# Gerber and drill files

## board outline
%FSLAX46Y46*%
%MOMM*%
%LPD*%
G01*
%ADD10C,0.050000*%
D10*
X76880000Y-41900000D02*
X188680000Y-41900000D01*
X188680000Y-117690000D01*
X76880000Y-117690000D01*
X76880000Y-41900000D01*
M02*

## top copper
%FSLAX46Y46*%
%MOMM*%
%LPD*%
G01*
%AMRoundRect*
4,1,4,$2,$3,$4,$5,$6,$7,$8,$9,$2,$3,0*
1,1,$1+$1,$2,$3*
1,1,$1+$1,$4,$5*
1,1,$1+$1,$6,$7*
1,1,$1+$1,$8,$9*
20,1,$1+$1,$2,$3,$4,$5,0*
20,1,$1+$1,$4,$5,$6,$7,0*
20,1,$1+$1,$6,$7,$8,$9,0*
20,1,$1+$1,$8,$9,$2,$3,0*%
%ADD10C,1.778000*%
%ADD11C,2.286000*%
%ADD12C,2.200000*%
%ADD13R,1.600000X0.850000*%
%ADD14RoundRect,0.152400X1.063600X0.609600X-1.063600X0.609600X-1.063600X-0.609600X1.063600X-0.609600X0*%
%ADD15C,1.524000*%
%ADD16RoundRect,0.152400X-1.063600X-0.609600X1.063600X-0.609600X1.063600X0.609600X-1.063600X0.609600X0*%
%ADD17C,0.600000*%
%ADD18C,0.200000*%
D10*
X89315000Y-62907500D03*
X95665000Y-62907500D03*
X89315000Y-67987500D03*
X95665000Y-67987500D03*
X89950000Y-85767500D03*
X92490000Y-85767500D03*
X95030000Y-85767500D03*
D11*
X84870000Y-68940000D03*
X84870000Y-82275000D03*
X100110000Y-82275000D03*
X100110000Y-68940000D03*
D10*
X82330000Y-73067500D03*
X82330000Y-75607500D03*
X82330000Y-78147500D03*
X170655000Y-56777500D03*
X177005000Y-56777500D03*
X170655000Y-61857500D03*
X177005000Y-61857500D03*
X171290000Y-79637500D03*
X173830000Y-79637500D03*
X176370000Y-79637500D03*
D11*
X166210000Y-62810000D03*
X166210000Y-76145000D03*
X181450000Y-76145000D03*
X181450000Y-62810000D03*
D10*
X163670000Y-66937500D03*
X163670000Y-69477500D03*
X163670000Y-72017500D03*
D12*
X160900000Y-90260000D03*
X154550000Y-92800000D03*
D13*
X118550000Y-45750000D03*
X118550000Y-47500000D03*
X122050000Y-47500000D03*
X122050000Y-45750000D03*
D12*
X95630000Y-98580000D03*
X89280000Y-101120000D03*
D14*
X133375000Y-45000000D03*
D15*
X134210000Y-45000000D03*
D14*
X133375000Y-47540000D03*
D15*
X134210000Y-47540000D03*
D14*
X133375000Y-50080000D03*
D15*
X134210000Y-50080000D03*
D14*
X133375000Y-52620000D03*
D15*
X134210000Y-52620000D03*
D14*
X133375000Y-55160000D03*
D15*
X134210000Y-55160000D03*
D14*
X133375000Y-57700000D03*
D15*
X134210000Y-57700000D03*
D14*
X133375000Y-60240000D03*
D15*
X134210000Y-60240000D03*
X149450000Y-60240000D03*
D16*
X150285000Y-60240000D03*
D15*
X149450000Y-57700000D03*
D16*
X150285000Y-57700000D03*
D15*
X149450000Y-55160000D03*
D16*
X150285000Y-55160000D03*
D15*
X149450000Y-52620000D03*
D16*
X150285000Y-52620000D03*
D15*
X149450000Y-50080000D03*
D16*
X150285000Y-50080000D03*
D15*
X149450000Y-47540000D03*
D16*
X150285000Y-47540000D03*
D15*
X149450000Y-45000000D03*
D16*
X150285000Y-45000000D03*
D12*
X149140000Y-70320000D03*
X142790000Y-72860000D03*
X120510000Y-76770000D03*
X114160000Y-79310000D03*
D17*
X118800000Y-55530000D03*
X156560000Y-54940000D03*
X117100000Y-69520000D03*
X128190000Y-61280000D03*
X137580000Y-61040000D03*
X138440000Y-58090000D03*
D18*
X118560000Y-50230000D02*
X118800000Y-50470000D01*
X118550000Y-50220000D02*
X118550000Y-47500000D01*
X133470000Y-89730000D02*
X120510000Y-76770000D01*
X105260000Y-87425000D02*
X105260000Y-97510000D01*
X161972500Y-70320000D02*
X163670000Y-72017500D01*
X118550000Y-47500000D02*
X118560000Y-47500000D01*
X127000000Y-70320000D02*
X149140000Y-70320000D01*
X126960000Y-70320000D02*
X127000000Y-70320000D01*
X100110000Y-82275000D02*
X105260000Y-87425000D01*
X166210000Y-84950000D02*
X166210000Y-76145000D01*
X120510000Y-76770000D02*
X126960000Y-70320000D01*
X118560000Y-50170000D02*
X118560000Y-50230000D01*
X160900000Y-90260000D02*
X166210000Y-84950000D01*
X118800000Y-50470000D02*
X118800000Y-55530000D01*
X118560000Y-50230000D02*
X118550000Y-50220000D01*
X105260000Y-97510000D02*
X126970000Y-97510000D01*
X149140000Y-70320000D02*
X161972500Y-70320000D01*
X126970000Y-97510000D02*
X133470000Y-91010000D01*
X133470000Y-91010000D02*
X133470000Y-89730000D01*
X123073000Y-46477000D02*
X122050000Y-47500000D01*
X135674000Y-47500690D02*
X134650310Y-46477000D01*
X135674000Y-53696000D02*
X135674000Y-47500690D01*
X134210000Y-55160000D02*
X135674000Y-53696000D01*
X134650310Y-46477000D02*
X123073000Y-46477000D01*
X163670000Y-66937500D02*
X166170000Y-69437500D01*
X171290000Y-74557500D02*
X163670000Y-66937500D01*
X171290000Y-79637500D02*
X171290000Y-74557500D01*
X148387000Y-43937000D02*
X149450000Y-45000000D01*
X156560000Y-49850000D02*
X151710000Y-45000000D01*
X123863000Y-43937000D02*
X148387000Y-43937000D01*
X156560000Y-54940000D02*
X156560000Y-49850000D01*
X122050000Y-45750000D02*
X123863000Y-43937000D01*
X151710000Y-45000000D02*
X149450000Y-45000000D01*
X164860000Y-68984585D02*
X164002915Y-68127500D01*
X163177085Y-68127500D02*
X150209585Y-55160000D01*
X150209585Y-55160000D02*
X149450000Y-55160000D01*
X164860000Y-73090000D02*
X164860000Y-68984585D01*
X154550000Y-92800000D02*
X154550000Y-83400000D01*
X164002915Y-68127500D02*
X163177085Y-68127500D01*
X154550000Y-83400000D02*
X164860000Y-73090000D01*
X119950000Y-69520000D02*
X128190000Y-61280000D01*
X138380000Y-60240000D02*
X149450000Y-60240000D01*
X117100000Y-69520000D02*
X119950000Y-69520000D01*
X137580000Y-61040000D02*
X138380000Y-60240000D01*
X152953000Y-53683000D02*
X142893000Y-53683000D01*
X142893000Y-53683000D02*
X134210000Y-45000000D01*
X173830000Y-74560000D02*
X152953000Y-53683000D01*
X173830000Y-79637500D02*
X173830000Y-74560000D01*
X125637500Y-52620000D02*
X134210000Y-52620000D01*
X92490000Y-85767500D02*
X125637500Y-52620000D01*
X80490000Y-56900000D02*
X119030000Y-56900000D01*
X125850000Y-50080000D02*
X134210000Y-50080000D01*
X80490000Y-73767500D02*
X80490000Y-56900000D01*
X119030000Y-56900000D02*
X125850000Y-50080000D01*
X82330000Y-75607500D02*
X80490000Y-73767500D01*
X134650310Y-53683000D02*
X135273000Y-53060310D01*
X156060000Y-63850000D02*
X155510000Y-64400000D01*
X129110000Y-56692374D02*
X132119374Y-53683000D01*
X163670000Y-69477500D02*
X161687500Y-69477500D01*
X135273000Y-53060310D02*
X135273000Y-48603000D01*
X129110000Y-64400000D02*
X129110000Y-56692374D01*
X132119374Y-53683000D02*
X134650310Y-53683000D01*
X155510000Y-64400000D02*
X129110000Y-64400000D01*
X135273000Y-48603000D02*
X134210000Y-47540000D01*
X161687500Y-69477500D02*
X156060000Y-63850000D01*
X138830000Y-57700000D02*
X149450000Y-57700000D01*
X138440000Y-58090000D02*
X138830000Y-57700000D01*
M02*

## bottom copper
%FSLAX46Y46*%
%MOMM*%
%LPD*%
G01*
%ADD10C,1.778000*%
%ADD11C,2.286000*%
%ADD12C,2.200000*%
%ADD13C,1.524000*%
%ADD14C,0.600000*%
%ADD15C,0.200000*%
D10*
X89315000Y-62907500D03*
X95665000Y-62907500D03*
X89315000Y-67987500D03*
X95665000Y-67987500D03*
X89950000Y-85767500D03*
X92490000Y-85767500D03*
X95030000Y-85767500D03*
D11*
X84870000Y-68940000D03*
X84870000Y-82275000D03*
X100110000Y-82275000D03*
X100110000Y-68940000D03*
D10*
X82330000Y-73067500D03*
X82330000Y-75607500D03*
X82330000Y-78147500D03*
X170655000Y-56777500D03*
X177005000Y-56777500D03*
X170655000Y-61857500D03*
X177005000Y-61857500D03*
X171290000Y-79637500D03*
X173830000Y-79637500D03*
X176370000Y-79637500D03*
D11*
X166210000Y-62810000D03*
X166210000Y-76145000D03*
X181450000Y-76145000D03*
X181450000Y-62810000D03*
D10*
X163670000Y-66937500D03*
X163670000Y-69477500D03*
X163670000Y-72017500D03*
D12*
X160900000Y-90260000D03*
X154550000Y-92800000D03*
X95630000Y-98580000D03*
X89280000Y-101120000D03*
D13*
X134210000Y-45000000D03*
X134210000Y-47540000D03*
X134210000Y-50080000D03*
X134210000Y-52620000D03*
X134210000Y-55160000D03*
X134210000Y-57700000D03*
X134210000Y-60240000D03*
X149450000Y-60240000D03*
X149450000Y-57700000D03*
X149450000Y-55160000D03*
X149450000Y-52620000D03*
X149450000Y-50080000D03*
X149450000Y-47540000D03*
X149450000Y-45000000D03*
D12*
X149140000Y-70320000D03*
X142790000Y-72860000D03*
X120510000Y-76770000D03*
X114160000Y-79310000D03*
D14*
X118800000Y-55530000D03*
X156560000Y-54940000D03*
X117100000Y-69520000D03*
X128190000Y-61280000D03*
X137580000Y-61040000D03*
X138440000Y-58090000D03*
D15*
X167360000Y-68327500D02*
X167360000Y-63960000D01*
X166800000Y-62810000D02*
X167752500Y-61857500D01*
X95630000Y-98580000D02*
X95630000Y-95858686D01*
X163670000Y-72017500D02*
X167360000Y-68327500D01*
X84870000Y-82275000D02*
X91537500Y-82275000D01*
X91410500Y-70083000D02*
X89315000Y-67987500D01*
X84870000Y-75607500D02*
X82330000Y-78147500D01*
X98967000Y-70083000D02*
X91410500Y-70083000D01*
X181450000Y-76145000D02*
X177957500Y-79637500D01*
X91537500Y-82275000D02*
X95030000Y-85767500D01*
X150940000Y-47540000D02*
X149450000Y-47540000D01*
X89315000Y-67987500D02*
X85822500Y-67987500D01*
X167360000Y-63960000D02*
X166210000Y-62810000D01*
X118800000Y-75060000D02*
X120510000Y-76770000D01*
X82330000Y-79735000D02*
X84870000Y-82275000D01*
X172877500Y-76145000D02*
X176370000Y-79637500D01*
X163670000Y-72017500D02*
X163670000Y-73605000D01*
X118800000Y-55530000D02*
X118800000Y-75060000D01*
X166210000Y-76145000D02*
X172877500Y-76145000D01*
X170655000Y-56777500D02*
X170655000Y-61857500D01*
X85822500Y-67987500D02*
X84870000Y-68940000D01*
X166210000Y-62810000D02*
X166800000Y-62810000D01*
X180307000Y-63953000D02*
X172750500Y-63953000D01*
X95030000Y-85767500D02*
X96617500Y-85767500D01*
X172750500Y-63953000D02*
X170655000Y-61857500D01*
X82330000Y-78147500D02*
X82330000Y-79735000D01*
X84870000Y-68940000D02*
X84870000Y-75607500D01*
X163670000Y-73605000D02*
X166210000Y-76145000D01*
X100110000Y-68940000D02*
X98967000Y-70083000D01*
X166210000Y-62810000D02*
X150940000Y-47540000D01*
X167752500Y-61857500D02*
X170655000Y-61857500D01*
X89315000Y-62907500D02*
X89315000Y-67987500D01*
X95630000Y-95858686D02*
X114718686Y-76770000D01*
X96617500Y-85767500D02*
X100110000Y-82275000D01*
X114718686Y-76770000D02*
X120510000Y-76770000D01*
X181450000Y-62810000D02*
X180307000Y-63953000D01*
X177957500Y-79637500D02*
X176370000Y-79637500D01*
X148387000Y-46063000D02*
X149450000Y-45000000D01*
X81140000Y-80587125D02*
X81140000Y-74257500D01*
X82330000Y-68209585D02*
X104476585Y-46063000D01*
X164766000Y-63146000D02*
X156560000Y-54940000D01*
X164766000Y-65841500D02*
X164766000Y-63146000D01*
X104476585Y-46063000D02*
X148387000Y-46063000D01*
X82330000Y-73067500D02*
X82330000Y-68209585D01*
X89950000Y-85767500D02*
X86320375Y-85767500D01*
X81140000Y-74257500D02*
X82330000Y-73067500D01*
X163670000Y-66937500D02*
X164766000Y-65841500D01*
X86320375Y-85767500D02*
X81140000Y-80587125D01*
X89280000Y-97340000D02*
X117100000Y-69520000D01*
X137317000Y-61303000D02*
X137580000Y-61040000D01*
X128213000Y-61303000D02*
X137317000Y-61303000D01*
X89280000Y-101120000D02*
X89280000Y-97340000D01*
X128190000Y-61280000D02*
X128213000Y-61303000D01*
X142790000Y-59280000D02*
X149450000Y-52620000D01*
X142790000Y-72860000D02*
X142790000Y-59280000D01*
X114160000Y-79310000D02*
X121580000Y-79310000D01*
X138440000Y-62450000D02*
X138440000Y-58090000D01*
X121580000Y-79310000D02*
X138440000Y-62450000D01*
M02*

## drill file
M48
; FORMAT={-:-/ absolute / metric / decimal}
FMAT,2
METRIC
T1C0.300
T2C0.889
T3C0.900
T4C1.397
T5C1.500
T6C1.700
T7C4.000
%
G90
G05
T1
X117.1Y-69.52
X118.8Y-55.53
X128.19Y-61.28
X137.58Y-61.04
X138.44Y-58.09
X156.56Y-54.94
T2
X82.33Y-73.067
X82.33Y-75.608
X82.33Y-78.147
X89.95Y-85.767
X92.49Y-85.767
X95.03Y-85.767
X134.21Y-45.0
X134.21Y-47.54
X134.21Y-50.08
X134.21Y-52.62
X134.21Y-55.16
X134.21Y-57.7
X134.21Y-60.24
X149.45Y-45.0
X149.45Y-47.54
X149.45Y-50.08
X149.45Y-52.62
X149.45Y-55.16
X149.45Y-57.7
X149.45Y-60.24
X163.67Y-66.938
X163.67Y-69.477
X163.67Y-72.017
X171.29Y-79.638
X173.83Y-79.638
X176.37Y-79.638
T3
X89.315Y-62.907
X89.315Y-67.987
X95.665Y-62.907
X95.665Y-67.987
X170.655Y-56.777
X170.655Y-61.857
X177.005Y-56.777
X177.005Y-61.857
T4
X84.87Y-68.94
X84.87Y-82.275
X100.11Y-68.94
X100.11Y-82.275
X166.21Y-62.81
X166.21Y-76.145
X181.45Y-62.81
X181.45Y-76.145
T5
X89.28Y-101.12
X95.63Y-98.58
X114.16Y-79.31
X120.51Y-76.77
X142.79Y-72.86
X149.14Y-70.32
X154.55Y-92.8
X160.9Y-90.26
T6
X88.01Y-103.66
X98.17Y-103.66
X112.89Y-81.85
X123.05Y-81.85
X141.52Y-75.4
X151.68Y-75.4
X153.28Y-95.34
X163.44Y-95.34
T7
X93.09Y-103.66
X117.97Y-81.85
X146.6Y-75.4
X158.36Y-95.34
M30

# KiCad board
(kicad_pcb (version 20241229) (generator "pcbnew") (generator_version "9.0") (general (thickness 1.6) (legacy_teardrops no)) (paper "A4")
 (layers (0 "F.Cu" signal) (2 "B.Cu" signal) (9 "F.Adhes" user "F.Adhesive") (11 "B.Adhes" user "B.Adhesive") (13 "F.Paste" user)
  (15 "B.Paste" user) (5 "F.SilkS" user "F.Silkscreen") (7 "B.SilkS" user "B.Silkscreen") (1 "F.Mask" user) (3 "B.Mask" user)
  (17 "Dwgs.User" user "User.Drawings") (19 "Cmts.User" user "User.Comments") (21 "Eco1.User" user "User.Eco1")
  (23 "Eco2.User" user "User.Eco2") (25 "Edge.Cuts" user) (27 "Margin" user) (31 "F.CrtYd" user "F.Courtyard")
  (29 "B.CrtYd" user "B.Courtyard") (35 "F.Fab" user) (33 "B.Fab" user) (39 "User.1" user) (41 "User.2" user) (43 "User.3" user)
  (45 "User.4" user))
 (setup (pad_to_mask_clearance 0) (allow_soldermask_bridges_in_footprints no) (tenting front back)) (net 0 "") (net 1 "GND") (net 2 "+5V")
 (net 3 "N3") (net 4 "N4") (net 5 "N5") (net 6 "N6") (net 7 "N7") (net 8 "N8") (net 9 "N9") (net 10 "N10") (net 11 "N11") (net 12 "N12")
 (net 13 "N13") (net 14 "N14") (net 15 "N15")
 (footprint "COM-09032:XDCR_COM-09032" (layer "F.Cu") (at 92.49 75.6075)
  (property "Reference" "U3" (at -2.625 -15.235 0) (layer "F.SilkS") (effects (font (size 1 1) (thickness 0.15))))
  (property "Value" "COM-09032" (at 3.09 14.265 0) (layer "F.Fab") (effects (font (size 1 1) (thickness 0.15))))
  (pad "B1A" thru_hole circle (at -3.175 -12.7) (size 1.778 1.778) (drill 0.9) (layers "*.Cu" "*.Mask") (remove_unused_layers no)
   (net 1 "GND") (solder_mask_margin 0.102))
  (pad "B1B" thru_hole circle (at 3.175 -12.7) (size 1.778 1.778) (drill 0.9) (layers "*.Cu" "*.Mask") (remove_unused_layers no)
   (solder_mask_margin 0.102))
  (pad "B2A" thru_hole circle (at -3.175 -7.62) (size 1.778 1.778) (drill 0.9) (layers "*.Cu" "*.Mask") (remove_unused_layers no)
   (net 1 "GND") (solder_mask_margin 0.102))
  (pad "B2B" thru_hole circle (at 3.175 -7.62) (size 1.778 1.778) (drill 0.9) (layers "*.Cu" "*.Mask") (remove_unused_layers no)
   (solder_mask_margin 0.102))
  (pad "H1" thru_hole circle (at -2.54 10.16) (size 1.778 1.778) (drill 0.889) (layers "*.Cu" "*.Mask") (remove_unused_layers no)
   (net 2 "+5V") (solder_mask_margin 0.102))
  (pad "H2" thru_hole circle (at 0 10.16) (size 1.778 1.778) (drill 0.889) (layers "*.Cu" "*.Mask") (remove_unused_layers no) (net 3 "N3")
   (solder_mask_margin 0.102))
  (pad "H3" thru_hole circle (at 2.54 10.16) (size 1.778 1.778) (drill 0.889) (layers "*.Cu" "*.Mask") (remove_unused_layers no)
   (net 1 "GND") (solder_mask_margin 0.102))
  (pad "S1" thru_hole circle (at -7.62 -6.6675) (size 2.286 2.286) (drill 1.397) (layers "*.Cu" "*.Mask") (remove_unused_layers no)
   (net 1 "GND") (solder_mask_margin 0.102))
  (pad "S2" thru_hole circle (at -7.62 6.6675) (size 2.286 2.286) (drill 1.397) (layers "*.Cu" "*.Mask") (remove_unused_layers no)
   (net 1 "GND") (solder_mask_margin 0.102))
  (pad "S3" thru_hole circle (at 7.62 6.6675) (size 2.286 2.286) (drill 1.397) (layers "*.Cu" "*.Mask") (remove_unused_layers no)
   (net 1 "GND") (solder_mask_margin 0.102))
  (pad "S4" thru_hole circle (at 7.62 -6.6675) (size 2.286 2.286) (drill 1.397) (layers "*.Cu" "*.Mask") (remove_unused_layers no)
   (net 1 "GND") (solder_mask_margin 0.102))
  (pad "V1" thru_hole circle (at -10.16 -2.54) (size 1.778 1.778) (drill 0.889) (layers "*.Cu" "*.Mask") (remove_unused_layers no)
   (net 2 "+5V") (solder_mask_margin 0.102))
  (pad "V2" thru_hole circle (at -10.16 0) (size 1.778 1.778) (drill 0.889) (layers "*.Cu" "*.Mask") (remove_unused_layers no) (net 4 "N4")
   (solder_mask_margin 0.102))
  (pad "V3" thru_hole circle (at -10.16 2.54) (size 1.778 1.778) (drill 0.889) (layers "*.Cu" "*.Mask") (remove_unused_layers no)
   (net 1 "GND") (solder_mask_margin 0.102)))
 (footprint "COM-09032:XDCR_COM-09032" (layer "F.Cu") (at 173.83 69.4775)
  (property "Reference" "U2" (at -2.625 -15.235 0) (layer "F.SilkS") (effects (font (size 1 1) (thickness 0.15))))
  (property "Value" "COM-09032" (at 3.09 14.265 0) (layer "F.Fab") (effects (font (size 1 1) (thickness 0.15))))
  (pad "B1A" thru_hole circle (at -3.175 -12.7) (size 1.778 1.778) (drill 0.9) (layers "*.Cu" "*.Mask") (remove_unused_layers no)
   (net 1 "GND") (solder_mask_margin 0.102))
  (pad "B1B" thru_hole circle (at 3.175 -12.7) (size 1.778 1.778) (drill 0.9) (layers "*.Cu" "*.Mask") (remove_unused_layers no)
   (solder_mask_margin 0.102))
  (pad "B2A" thru_hole circle (at -3.175 -7.62) (size 1.778 1.778) (drill 0.9) (layers "*.Cu" "*.Mask") (remove_unused_layers no)
   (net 1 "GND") (solder_mask_margin 0.102))
  (pad "B2B" thru_hole circle (at 3.175 -7.62) (size 1.778 1.778) (drill 0.9) (layers "*.Cu" "*.Mask") (remove_unused_layers no)
   (solder_mask_margin 0.102))
  (pad "H1" thru_hole circle (at -2.54 10.16) (size 1.778 1.778) (drill 0.889) (layers "*.Cu" "*.Mask") (remove_unused_layers no)
   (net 2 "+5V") (solder_mask_margin 0.102))
  (pad "H2" thru_hole circle (at 0 10.16) (size 1.778 1.778) (drill 0.889) (layers "*.Cu" "*.Mask") (remove_unused_layers no) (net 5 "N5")
   (solder_mask_margin 0.102))
  (pad "H3" thru_hole circle (at 2.54 10.16) (size 1.778 1.778) (drill 0.889) (layers "*.Cu" "*.Mask") (remove_unused_layers no)
   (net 1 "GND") (solder_mask_margin 0.102))
  (pad "S1" thru_hole circle (at -7.62 -6.6675) (size 2.286 2.286) (drill 1.397) (layers "*.Cu" "*.Mask") (remove_unused_layers no)
   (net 1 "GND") (solder_mask_margin 0.102))
  (pad "S2" thru_hole circle (at -7.62 6.6675) (size 2.286 2.286) (drill 1.397) (layers "*.Cu" "*.Mask") (remove_unused_layers no)
   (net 1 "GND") (solder_mask_margin 0.102))
  (pad "S3" thru_hole circle (at 7.62 6.6675) (size 2.286 2.286) (drill 1.397) (layers "*.Cu" "*.Mask") (remove_unused_layers no)
   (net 1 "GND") (solder_mask_margin 0.102))
  (pad "S4" thru_hole circle (at 7.62 -6.6675) (size 2.286 2.286) (drill 1.397) (layers "*.Cu" "*.Mask") (remove_unused_layers no)
   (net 1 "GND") (solder_mask_margin 0.102))
  (pad "V1" thru_hole circle (at -10.16 -2.54) (size 1.778 1.778) (drill 0.889) (layers "*.Cu" "*.Mask") (remove_unused_layers no)
   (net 2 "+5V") (solder_mask_margin 0.102))
  (pad "V2" thru_hole circle (at -10.16 0) (size 1.778 1.778) (drill 0.889) (layers "*.Cu" "*.Mask") (remove_unused_layers no) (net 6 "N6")
   (solder_mask_margin 0.102))
  (pad "V3" thru_hole circle (at -10.16 2.54) (size 1.778 1.778) (drill 0.889) (layers "*.Cu" "*.Mask") (remove_unused_layers no)
   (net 1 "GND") (solder_mask_margin 0.102)))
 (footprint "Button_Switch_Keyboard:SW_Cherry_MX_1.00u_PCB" (layer "F.Cu") (at 160.9 90.26)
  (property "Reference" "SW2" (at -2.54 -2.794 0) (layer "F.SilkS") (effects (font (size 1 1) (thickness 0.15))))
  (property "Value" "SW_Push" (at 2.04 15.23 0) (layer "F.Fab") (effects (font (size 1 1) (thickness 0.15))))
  (pad "" np_thru_hole circle (at -7.62 5.08) (size 1.7 1.7) (drill 1.7) (layers "*.Cu" "*.Mask"))
  (pad "" np_thru_hole circle (at -2.54 5.08) (size 4 4) (drill 4) (layers "*.Cu" "*.Mask"))
  (pad "" np_thru_hole circle (at 2.54 5.08) (size 1.7 1.7) (drill 1.7) (layers "*.Cu" "*.Mask"))
  (pad "1" thru_hole circle (at 0 0) (size 2.2 2.2) (drill 1.5) (layers "*.Cu" "*.Mask") (remove_unused_layers no) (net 1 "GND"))
  (pad "2" thru_hole circle (at -6.35 2.54) (size 2.2 2.2) (drill 1.5) (layers "*.Cu" "*.Mask") (remove_unused_layers no) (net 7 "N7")))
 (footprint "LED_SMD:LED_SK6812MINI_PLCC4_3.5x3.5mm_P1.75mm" (layer "F.Cu") (at 120.3 46.625)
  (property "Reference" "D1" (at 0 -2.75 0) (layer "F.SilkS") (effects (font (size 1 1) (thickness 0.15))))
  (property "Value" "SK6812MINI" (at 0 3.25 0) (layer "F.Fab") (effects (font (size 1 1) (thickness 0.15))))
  (pad "1" smd rect (at -1.75 -0.875) (size 1.6 0.85) (layers "F.Cu" "F.Mask" "F.Paste") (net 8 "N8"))
  (pad "2" smd rect (at -1.75 0.875) (size 1.6 0.85) (layers "F.Cu" "F.Mask" "F.Paste") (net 1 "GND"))
  (pad "3" smd rect (at 1.75 0.875) (size 1.6 0.85) (layers "F.Cu" "F.Mask" "F.Paste") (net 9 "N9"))
  (pad "4" smd rect (at 1.75 -0.875) (size 1.6 0.85) (layers "F.Cu" "F.Mask" "F.Paste") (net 2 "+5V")))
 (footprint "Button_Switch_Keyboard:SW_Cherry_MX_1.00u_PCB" (layer "F.Cu") (at 95.63 98.58)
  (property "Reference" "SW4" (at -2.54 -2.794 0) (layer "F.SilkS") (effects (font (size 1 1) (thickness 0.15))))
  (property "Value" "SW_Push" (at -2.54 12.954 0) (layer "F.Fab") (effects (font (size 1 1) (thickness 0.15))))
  (pad "" np_thru_hole circle (at -7.62 5.08) (size 1.7 1.7) (drill 1.7) (layers "*.Cu" "*.Mask"))
  (pad "" np_thru_hole circle (at -2.54 5.08) (size 4 4) (drill 4) (layers "*.Cu" "*.Mask"))
  (pad "" np_thru_hole circle (at 2.54 5.08) (size 1.7 1.7) (drill 1.7) (layers "*.Cu" "*.Mask"))
  (pad "1" thru_hole circle (at 0 0) (size 2.2 2.2) (drill 1.5) (layers "*.Cu" "*.Mask") (remove_unused_layers no) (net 1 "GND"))
  (pad "2" thru_hole circle (at -6.35 2.54) (size 2.2 2.2) (drill 1.5) (layers "*.Cu" "*.Mask") (remove_unused_layers no) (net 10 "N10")))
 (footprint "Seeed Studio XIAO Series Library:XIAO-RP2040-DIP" (layer "F.Cu") (at 141.83 52.62)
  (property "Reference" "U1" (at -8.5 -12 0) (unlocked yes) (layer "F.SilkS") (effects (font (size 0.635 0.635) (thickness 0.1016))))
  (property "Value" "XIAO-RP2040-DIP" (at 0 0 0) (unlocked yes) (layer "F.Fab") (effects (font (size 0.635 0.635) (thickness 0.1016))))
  (pad "1" smd roundrect (at -8.455 -7.62 180) (size 2.432 1.524) (layers "F.Cu" "F.Mask") (roundrect_rratio 0.1) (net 5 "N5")
   (thermal_bridge_angle 45))
  (pad "1" thru_hole circle (at -7.62 -7.62 180) (size 1.524 1.524) (drill 0.889) (layers "*.Cu" "*.Mask") (remove_unused_layers no)
   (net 5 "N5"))
  (pad "2" smd roundrect (at -8.455 -5.08 180) (size 2.432 1.524) (layers "F.Cu" "F.Mask") (roundrect_rratio 0.1) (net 6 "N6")
   (thermal_bridge_angle 45))
  (pad "2" thru_hole circle (at -7.62 -5.08 180) (size 1.524 1.524) (drill 0.889) (layers "*.Cu" "*.Mask") (remove_unused_layers no)
   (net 6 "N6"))
  (pad "3" smd roundrect (at -8.455 -2.54 180) (size 2.432 1.524) (layers "F.Cu" "F.Mask") (roundrect_rratio 0.1) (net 4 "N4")
   (thermal_bridge_angle 45))
  (pad "3" thru_hole circle (at -7.62 -2.54 180) (size 1.524 1.524) (drill 0.889) (layers "*.Cu" "*.Mask") (remove_unused_layers no)
   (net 4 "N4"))
  (pad "4" smd roundrect (at -8.455 0 180) (size 2.432 1.524) (layers "F.Cu" "F.Mask") (roundrect_rratio 0.1) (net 3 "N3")
   (thermal_bridge_angle 45))
  (pad "4" thru_hole circle (at -7.62 0 180) (size 1.524 1.524) (drill 0.889) (layers "*.Cu" "*.Mask") (remove_unused_layers no)
   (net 3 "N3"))
  (pad "5" smd roundrect (at -8.455 2.54 180) (size 2.432 1.524) (layers "F.Cu" "F.Mask") (roundrect_rratio 0.1) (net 9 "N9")
   (thermal_bridge_angle 45))
  (pad "5" thru_hole circle (at -7.62 2.54 180) (size 1.524 1.524) (drill 0.889) (layers "*.Cu" "*.Mask") (remove_unused_layers no)
   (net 9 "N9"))
  (pad "6" smd roundrect (at -8.455 5.08 180) (size 2.432 1.524) (layers "F.Cu" "F.Mask") (roundrect_rratio 0.1) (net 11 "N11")
   (thermal_bridge_angle 45))
  (pad "6" thru_hole circle (at -7.62 5.08 180) (size 1.524 1.524) (drill 0.889) (layers "*.Cu" "*.Mask") (remove_unused_layers no)
   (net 11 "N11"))
  (pad "7" smd roundrect (at -8.455 7.62 180) (size 2.432 1.524) (layers "F.Cu" "F.Mask") (roundrect_rratio 0.1) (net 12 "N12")
   (thermal_bridge_angle 45))
  (pad "7" thru_hole circle (at -7.62 7.62 180) (size 1.524 1.524) (drill 0.889) (layers "*.Cu" "*.Mask") (remove_unused_layers no)
   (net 12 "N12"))
  (pad "8" thru_hole circle (at 7.62 7.62) (size 1.524 1.524) (drill 0.889) (layers "*.Cu" "*.Mask") (remove_unused_layers no)
   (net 10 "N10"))
  (pad "8" smd roundrect (at 8.455 7.62) (size 2.432 1.524) (layers "F.Cu" "F.Mask") (roundrect_rratio 0.1) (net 10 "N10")
   (thermal_bridge_angle 45))
  (pad "9" thru_hole circle (at 7.62 5.08) (size 1.524 1.524) (drill 0.889) (layers "*.Cu" "*.Mask") (remove_unused_layers no)
   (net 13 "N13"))
  (pad "9" smd roundrect (at 8.455 5.08) (size 2.432 1.524) (layers "F.Cu" "F.Mask") (roundrect_rratio 0.1) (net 13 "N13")
   (thermal_bridge_angle 45))
  (pad "10" thru_hole circle (at 7.62 2.54) (size 1.524 1.524) (drill 0.889) (layers "*.Cu" "*.Mask") (remove_unused_layers no) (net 7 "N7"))
  (pad "10" smd roundrect (at 8.455 2.54) (size 2.432 1.524) (layers "F.Cu" "F.Mask") (roundrect_rratio 0.1) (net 7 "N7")
   (thermal_bridge_angle 45))
  (pad "11" thru_hole circle (at 7.62 0) (size 1.524 1.524) (drill 0.889) (layers "*.Cu" "*.Mask") (remove_unused_layers no) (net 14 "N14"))
  (pad "11" smd roundrect (at 8.455 0) (size 2.432 1.524) (layers "F.Cu" "F.Mask") (roundrect_rratio 0.1) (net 14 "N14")
   (thermal_bridge_angle 45))
  (pad "12" thru_hole circle (at 7.62 -2.54) (size 1.524 1.524) (drill 0.889) (layers "*.Cu" "*.Mask") (remove_unused_layers no)
   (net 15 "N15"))
  (pad "12" smd roundrect (at 8.455 -2.54) (size 2.432 1.524) (layers "F.Cu" "F.Mask") (roundrect_rratio 0.1) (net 15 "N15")
   (thermal_bridge_angle 45))
  (pad "13" thru_hole circle (at 7.62 -5.08) (size 1.524 1.524) (drill 0.889) (layers "*.Cu" "*.Mask") (remove_unused_layers no)
   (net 1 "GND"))
  (pad "13" smd roundrect (at 8.455 -5.08) (size 2.432 1.524) (layers "F.Cu" "F.Mask") (roundrect_rratio 0.1) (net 1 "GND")
   (thermal_bridge_angle 45))
  (pad "14" thru_hole circle (at 7.62 -7.62) (size 1.524 1.524) (drill 0.889) (layers "*.Cu" "*.Mask") (remove_unused_layers no)
   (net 2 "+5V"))
  (pad "14" smd roundrect (at 8.455 -7.62) (size 2.432 1.524) (layers "F.Cu" "F.Mask") (roundrect_rratio 0.1) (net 2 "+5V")
   (thermal_bridge_angle 45)))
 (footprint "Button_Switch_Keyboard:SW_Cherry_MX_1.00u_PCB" (layer "F.Cu") (at 149.14 70.32)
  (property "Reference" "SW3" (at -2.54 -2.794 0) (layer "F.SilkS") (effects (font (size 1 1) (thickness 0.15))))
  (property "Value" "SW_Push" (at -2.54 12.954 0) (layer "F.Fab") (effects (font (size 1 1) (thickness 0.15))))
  (pad "" np_thru_hole circle (at -7.62 5.08) (size 1.7 1.7) (drill 1.7) (layers "*.Cu" "*.Mask"))
  (pad "" np_thru_hole circle (at -2.54 5.08) (size 4 4) (drill 4) (layers "*.Cu" "*.Mask"))
  (pad "" np_thru_hole circle (at 2.54 5.08) (size 1.7 1.7) (drill 1.7) (layers "*.Cu" "*.Mask"))
  (pad "1" thru_hole circle (at 0 0) (size 2.2 2.2) (drill 1.5) (layers "*.Cu" "*.Mask") (remove_unused_layers no) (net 1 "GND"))
  (pad "2" thru_hole circle (at -6.35 2.54) (size 2.2 2.2) (drill 1.5) (layers "*.Cu" "*.Mask") (remove_unused_layers no) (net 14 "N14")))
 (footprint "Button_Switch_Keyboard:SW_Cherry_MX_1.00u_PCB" (layer "F.Cu") (at 120.51 76.77)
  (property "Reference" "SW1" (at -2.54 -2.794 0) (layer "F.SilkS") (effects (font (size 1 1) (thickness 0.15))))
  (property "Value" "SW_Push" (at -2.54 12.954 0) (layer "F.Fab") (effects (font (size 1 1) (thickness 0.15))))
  (pad "" np_thru_hole circle (at -7.62 5.08) (size 1.7 1.7) (drill 1.7) (layers "*.Cu" "*.Mask"))
  (pad "" np_thru_hole circle (at -2.54 5.08) (size 4 4) (drill 4) (layers "*.Cu" "*.Mask"))
  (pad "" np_thru_hole circle (at 2.54 5.08) (size 1.7 1.7) (drill 1.7) (layers "*.Cu" "*.Mask"))
  (pad "1" thru_hole circle (at 0 0) (size 2.2 2.2) (drill 1.5) (layers "*.Cu" "*.Mask") (remove_unused_layers no) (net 1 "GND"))
  (pad "2" thru_hole circle (at -6.35 2.54) (size 2.2 2.2) (drill 1.5) (layers "*.Cu" "*.Mask") (remove_unused_layers no) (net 13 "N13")))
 (gr_rect (start 76.88 41.9) (end 188.68 117.69) (stroke (width 0.05) (type default)) (fill no) (layer "Edge.Cuts"))
 (segment (start 118.56 50.23) (end 118.8 50.47) (width 0.2) (layer "F.Cu") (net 1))
 (segment (start 118.55 50.22) (end 118.55 47.5) (width 0.2) (layer "F.Cu") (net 1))
 (segment (start 133.47 89.73) (end 120.51 76.77) (width 0.2) (layer "F.Cu") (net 1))
 (segment (start 105.26 87.425) (end 105.26 97.51) (width 0.2) (layer "F.Cu") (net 1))
 (segment (start 161.9725 70.32) (end 163.67 72.0175) (width 0.2) (layer "F.Cu") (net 1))
 (segment (start 118.55 47.5) (end 118.56 47.5) (width 0.2) (layer "F.Cu") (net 1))
 (segment (start 127 70.32) (end 149.14 70.32) (width 0.2) (layer "F.Cu") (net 1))
 (segment (start 126.96 70.32) (end 127 70.32) (width 0.2) (layer "F.Cu") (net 1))
 (segment (start 100.11 82.275) (end 105.26 87.425) (width 0.2) (layer "F.Cu") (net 1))
 (segment (start 166.21 84.95) (end 166.21 76.145) (width 0.2) (layer "F.Cu") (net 1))
 (segment (start 120.51 76.77) (end 126.96 70.32) (width 0.2) (layer "F.Cu") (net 1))
 (segment (start 118.56 50.17) (end 118.56 50.23) (width 0.2) (layer "F.Cu") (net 1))
 (segment (start 160.9 90.26) (end 166.21 84.95) (width 0.2) (layer "F.Cu") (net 1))
 (segment (start 118.8 50.47) (end 118.8 55.53) (width 0.2) (layer "F.Cu") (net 1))
 (segment (start 118.56 50.23) (end 118.55 50.22) (width 0.2) (layer "F.Cu") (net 1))
 (segment (start 105.26 97.51) (end 126.97 97.51) (width 0.2) (layer "F.Cu") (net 1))
 (segment (start 149.14 70.32) (end 161.9725 70.32) (width 0.2) (layer "F.Cu") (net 1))
 (segment (start 126.97 97.51) (end 133.47 91.01) (width 0.2) (layer "F.Cu") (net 1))
 (segment (start 133.47 91.01) (end 133.47 89.73) (width 0.2) (layer "F.Cu") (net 1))
 (via (at 118.8 55.53) (size 0.6) (drill 0.3) (layers "F.Cu" "B.Cu") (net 1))
 (segment (start 167.36 68.3275) (end 167.36 63.96) (width 0.2) (layer "B.Cu") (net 1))
 (segment (start 166.8 62.81) (end 167.7525 61.8575) (width 0.2) (layer "B.Cu") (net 1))
 (segment (start 95.63 98.58) (end 95.63 95.858686) (width 0.2) (layer "B.Cu") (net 1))
 (segment (start 163.67 72.0175) (end 167.36 68.3275) (width 0.2) (layer "B.Cu") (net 1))
 (segment (start 84.87 82.275) (end 91.5375 82.275) (width 0.2) (layer "B.Cu") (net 1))
 (segment (start 91.4105 70.083) (end 89.315 67.9875) (width 0.2) (layer "B.Cu") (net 1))
 (segment (start 84.87 75.6075) (end 82.33 78.1475) (width 0.2) (layer "B.Cu") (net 1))
 (segment (start 98.967 70.083) (end 91.4105 70.083) (width 0.2) (layer "B.Cu") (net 1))
 (segment (start 181.45 76.145) (end 177.9575 79.6375) (width 0.2) (layer "B.Cu") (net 1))
 (segment (start 91.5375 82.275) (end 95.03 85.7675) (width 0.2) (layer "B.Cu") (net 1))
 (segment (start 150.94 47.54) (end 149.45 47.54) (width 0.2) (layer "B.Cu") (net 1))
 (segment (start 89.315 67.9875) (end 85.8225 67.9875) (width 0.2) (layer "B.Cu") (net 1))
 (segment (start 167.36 63.96) (end 166.21 62.81) (width 0.2) (layer "B.Cu") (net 1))
 (segment (start 118.8 75.06) (end 120.51 76.77) (width 0.2) (layer "B.Cu") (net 1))
 (segment (start 82.33 79.735) (end 84.87 82.275) (width 0.2) (layer "B.Cu") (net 1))
 (segment (start 172.8775 76.145) (end 176.37 79.6375) (width 0.2) (layer "B.Cu") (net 1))
 (segment (start 163.67 72.0175) (end 163.67 73.605) (width 0.2) (layer "B.Cu") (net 1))
 (segment (start 118.8 55.53) (end 118.8 75.06) (width 0.2) (layer "B.Cu") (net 1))
 (segment (start 166.21 76.145) (end 172.8775 76.145) (width 0.2) (layer "B.Cu") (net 1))
 (segment (start 170.655 56.7775) (end 170.655 61.8575) (width 0.2) (layer "B.Cu") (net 1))
 (segment (start 85.8225 67.9875) (end 84.87 68.94) (width 0.2) (layer "B.Cu") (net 1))
 (segment (start 166.21 62.81) (end 166.8 62.81) (width 0.2) (layer "B.Cu") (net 1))
 (segment (start 180.307 63.953) (end 172.7505 63.953) (width 0.2) (layer "B.Cu") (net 1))
 (segment (start 95.03 85.7675) (end 96.6175 85.7675) (width 0.2) (layer "B.Cu") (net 1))
 (segment (start 172.7505 63.953) (end 170.655 61.8575) (width 0.2) (layer "B.Cu") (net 1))
 (segment (start 82.33 78.1475) (end 82.33 79.735) (width 0.2) (layer "B.Cu") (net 1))
 (segment (start 84.87 68.94) (end 84.87 75.6075) (width 0.2) (layer "B.Cu") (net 1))
 (segment (start 163.67 73.605) (end 166.21 76.145) (width 0.2) (layer "B.Cu") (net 1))
 (segment (start 100.11 68.94) (end 98.967 70.083) (width 0.2) (layer "B.Cu") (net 1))
 (segment (start 166.21 62.81) (end 150.94 47.54) (width 0.2) (layer "B.Cu") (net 1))
 (segment (start 167.7525 61.8575) (end 170.655 61.8575) (width 0.2) (layer "B.Cu") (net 1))
 (segment (start 89.315 62.9075) (end 89.315 67.9875) (width 0.2) (layer "B.Cu") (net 1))
 (segment (start 95.63 95.858686) (end 114.718686 76.77) (width 0.2) (layer "B.Cu") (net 1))
 (segment (start 96.6175 85.7675) (end 100.11 82.275) (width 0.2) (layer "B.Cu") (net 1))
 (segment (start 114.718686 76.77) (end 120.51 76.77) (width 0.2) (layer "B.Cu") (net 1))
 (segment (start 181.45 62.81) (end 180.307 63.953) (width 0.2) (layer "B.Cu") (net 1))
 (segment (start 177.9575 79.6375) (end 176.37 79.6375) (width 0.2) (layer "B.Cu") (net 1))
 (segment (start 123.073 46.477) (end 122.05 47.5) (width 0.2) (layer "F.Cu") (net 9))
 (segment (start 135.674 47.50069) (end 134.65031 46.477) (width 0.2) (layer "F.Cu") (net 9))
 (segment (start 135.674 53.696) (end 135.674 47.50069) (width 0.2) (layer "F.Cu") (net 9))
 (segment (start 134.21 55.16) (end 135.674 53.696) (width 0.2) (layer "F.Cu") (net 9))
 (segment (start 134.65031 46.477) (end 123.073 46.477) (width 0.2) (layer "F.Cu") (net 9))
 (segment (start 163.67 66.9375) (end 166.17 69.4375) (width 0.2) (layer "F.Cu") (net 2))
 (segment (start 171.29 74.5575) (end 163.67 66.9375) (width 0.2) (layer "F.Cu") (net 2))
 (segment (start 171.29 79.6375) (end 171.29 74.5575) (width 0.2) (layer "F.Cu") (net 2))
 (segment (start 148.387 43.937) (end 149.45 45) (width 0.2) (layer "F.Cu") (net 2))
 (segment (start 156.56 49.85) (end 151.71 45) (width 0.2) (layer "F.Cu") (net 2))
 (segment (start 123.863 43.937) (end 148.387 43.937) (width 0.2) (layer "F.Cu") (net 2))
 (segment (start 156.56 54.94) (end 156.56 49.85) (width 0.2) (layer "F.Cu") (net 2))
 (segment (start 122.05 45.75) (end 123.863 43.937) (width 0.2) (layer "F.Cu") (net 2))
 (segment (start 151.71 45) (end 149.45 45) (width 0.2) (layer "F.Cu") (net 2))
 (via (at 156.56 54.94) (size 0.6) (drill 0.3) (layers "F.Cu" "B.Cu") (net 2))
 (segment (start 148.387 46.063) (end 149.45 45) (width 0.2) (layer "B.Cu") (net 2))
 (segment (start 81.14 80.587125) (end 81.14 74.2575) (width 0.2) (layer "B.Cu") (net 2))
 (segment (start 82.33 68.209585) (end 104.476585 46.063) (width 0.2) (layer "B.Cu") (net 2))
 (segment (start 164.766 63.146) (end 156.56 54.94) (width 0.2) (layer "B.Cu") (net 2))
 (segment (start 164.766 65.8415) (end 164.766 63.146) (width 0.2) (layer "B.Cu") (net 2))
 (segment (start 104.476585 46.063) (end 148.387 46.063) (width 0.2) (layer "B.Cu") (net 2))
 (segment (start 82.33 73.0675) (end 82.33 68.209585) (width 0.2) (layer "B.Cu") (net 2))
 (segment (start 89.95 85.7675) (end 86.320375 85.7675) (width 0.2) (layer "B.Cu") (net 2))
 (segment (start 81.14 74.2575) (end 82.33 73.0675) (width 0.2) (layer "B.Cu") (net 2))
 (segment (start 163.67 66.9375) (end 164.766 65.8415) (width 0.2) (layer "B.Cu") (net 2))
 (segment (start 86.320375 85.7675) (end 81.14 80.587125) (width 0.2) (layer "B.Cu") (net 2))
 (segment (start 164.86 68.984585) (end 164.002915 68.1275) (width 0.2) (layer "F.Cu") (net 7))
 (segment (start 163.177085 68.1275) (end 150.209585 55.16) (width 0.2) (layer "F.Cu") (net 7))
 (segment (start 150.209585 55.16) (end 149.45 55.16) (width 0.2) (layer "F.Cu") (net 7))
 (segment (start 164.86 73.09) (end 164.86 68.984585) (width 0.2) (layer "F.Cu") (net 7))
 (segment (start 154.55 92.8) (end 154.55 83.4) (width 0.2) (layer "F.Cu") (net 7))
 (segment (start 164.002915 68.1275) (end 163.177085 68.1275) (width 0.2) (layer "F.Cu") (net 7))
 (segment (start 154.55 83.4) (end 164.86 73.09) (width 0.2) (layer "F.Cu") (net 7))
 (segment (start 119.95 69.52) (end 128.19 61.28) (width 0.2) (layer "F.Cu") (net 10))
 (segment (start 138.38 60.24) (end 149.45 60.24) (width 0.2) (layer "F.Cu") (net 10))
 (segment (start 117.1 69.52) (end 119.95 69.52) (width 0.2) (layer "F.Cu") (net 10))
 (segment (start 137.58 61.04) (end 138.38 60.24) (width 0.2) (layer "F.Cu") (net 10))
 (via (at 117.1 69.52) (size 0.6) (drill 0.3) (layers "F.Cu" "B.Cu") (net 10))
 (via (at 128.19 61.28) (size 0.6) (drill 0.3) (layers "F.Cu" "B.Cu") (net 10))
 (via (at 137.58 61.04) (size 0.6) (drill 0.3) (layers "F.Cu" "B.Cu") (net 10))
 (segment (start 89.28 97.34) (end 117.1 69.52) (width 0.2) (layer "B.Cu") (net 10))
 (segment (start 137.317 61.303) (end 137.58 61.04) (width 0.2) (layer "B.Cu") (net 10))
 (segment (start 128.213 61.303) (end 137.317 61.303) (width 0.2) (layer "B.Cu") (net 10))
 (segment (start 89.28 101.12) (end 89.28 97.34) (width 0.2) (layer "B.Cu") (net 10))
 (segment (start 128.19 61.28) (end 128.213 61.303) (width 0.2) (layer "B.Cu") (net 10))
 (segment (start 152.953 53.683) (end 142.893 53.683) (width 0.2) (layer "F.Cu") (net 5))
 (segment (start 142.893 53.683) (end 134.21 45) (width 0.2) (layer "F.Cu") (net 5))
 (segment (start 173.83 74.56) (end 152.953 53.683) (width 0.2) (layer "F.Cu") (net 5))
 (segment (start 173.83 79.6375) (end 173.83 74.56) (width 0.2) (layer "F.Cu") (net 5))
 (segment (start 142.79 59.28) (end 149.45 52.62) (width 0.2) (layer "B.Cu") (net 14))
 (segment (start 142.79 72.86) (end 142.79 59.28) (width 0.2) (layer "B.Cu") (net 14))
 (segment (start 125.6375 52.62) (end 134.21 52.62) (width 0.2) (layer "F.Cu") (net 3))
 (segment (start 92.49 85.7675) (end 125.6375 52.62) (width 0.2) (layer "F.Cu") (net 3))
 (segment (start 80.49 56.9) (end 119.03 56.9) (width 0.2) (layer "F.Cu") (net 4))
 (segment (start 125.85 50.08) (end 134.21 50.08) (width 0.2) (layer "F.Cu") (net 4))
 (segment (start 80.49 73.7675) (end 80.49 56.9) (width 0.2) (layer "F.Cu") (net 4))
 (segment (start 119.03 56.9) (end 125.85 50.08) (width 0.2) (layer "F.Cu") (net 4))
 (segment (start 82.33 75.6075) (end 80.49 73.7675) (width 0.2) (layer "F.Cu") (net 4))
 (segment (start 134.65031 53.683) (end 135.273 53.06031) (width 0.2) (layer "F.Cu") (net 6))
 (segment (start 156.06 63.85) (end 155.51 64.4) (width 0.2) (layer "F.Cu") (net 6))
 (segment (start 129.11 56.692374) (end 132.119374 53.683) (width 0.2) (layer "F.Cu") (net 6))
 (segment (start 163.67 69.4775) (end 161.6875 69.4775) (width 0.2) (layer "F.Cu") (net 6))
 (segment (start 135.273 53.06031) (end 135.273 48.603) (width 0.2) (layer "F.Cu") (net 6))
 (segment (start 129.11 64.4) (end 129.11 56.692374) (width 0.2) (layer "F.Cu") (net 6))
 (segment (start 132.119374 53.683) (end 134.65031 53.683) (width 0.2) (layer "F.Cu") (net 6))
 (segment (start 155.51 64.4) (end 129.11 64.4) (width 0.2) (layer "F.Cu") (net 6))
 (segment (start 135.273 48.603) (end 134.21 47.54) (width 0.2) (layer "F.Cu") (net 6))
 (segment (start 161.6875 69.4775) (end 156.06 63.85) (width 0.2) (layer "F.Cu") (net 6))
 (segment (start 138.83 57.7) (end 149.45 57.7) (width 0.2) (layer "F.Cu") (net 13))
 (segment (start 138.44 58.09) (end 138.83 57.7) (width 0.2) (layer "F.Cu") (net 13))
 (via (at 138.44 58.09) (size 0.6) (drill 0.3) (layers "F.Cu" "B.Cu") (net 13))
 (segment (start 114.16 79.31) (end 121.58 79.31) (width 0.2) (layer "B.Cu") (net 13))
 (segment (start 138.44 62.45) (end 138.44 58.09) (width 0.2) (layer "B.Cu") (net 13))
 (segment (start 121.58 79.31) (end 138.44 62.45) (width 0.2) (layer "B.Cu") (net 13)))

